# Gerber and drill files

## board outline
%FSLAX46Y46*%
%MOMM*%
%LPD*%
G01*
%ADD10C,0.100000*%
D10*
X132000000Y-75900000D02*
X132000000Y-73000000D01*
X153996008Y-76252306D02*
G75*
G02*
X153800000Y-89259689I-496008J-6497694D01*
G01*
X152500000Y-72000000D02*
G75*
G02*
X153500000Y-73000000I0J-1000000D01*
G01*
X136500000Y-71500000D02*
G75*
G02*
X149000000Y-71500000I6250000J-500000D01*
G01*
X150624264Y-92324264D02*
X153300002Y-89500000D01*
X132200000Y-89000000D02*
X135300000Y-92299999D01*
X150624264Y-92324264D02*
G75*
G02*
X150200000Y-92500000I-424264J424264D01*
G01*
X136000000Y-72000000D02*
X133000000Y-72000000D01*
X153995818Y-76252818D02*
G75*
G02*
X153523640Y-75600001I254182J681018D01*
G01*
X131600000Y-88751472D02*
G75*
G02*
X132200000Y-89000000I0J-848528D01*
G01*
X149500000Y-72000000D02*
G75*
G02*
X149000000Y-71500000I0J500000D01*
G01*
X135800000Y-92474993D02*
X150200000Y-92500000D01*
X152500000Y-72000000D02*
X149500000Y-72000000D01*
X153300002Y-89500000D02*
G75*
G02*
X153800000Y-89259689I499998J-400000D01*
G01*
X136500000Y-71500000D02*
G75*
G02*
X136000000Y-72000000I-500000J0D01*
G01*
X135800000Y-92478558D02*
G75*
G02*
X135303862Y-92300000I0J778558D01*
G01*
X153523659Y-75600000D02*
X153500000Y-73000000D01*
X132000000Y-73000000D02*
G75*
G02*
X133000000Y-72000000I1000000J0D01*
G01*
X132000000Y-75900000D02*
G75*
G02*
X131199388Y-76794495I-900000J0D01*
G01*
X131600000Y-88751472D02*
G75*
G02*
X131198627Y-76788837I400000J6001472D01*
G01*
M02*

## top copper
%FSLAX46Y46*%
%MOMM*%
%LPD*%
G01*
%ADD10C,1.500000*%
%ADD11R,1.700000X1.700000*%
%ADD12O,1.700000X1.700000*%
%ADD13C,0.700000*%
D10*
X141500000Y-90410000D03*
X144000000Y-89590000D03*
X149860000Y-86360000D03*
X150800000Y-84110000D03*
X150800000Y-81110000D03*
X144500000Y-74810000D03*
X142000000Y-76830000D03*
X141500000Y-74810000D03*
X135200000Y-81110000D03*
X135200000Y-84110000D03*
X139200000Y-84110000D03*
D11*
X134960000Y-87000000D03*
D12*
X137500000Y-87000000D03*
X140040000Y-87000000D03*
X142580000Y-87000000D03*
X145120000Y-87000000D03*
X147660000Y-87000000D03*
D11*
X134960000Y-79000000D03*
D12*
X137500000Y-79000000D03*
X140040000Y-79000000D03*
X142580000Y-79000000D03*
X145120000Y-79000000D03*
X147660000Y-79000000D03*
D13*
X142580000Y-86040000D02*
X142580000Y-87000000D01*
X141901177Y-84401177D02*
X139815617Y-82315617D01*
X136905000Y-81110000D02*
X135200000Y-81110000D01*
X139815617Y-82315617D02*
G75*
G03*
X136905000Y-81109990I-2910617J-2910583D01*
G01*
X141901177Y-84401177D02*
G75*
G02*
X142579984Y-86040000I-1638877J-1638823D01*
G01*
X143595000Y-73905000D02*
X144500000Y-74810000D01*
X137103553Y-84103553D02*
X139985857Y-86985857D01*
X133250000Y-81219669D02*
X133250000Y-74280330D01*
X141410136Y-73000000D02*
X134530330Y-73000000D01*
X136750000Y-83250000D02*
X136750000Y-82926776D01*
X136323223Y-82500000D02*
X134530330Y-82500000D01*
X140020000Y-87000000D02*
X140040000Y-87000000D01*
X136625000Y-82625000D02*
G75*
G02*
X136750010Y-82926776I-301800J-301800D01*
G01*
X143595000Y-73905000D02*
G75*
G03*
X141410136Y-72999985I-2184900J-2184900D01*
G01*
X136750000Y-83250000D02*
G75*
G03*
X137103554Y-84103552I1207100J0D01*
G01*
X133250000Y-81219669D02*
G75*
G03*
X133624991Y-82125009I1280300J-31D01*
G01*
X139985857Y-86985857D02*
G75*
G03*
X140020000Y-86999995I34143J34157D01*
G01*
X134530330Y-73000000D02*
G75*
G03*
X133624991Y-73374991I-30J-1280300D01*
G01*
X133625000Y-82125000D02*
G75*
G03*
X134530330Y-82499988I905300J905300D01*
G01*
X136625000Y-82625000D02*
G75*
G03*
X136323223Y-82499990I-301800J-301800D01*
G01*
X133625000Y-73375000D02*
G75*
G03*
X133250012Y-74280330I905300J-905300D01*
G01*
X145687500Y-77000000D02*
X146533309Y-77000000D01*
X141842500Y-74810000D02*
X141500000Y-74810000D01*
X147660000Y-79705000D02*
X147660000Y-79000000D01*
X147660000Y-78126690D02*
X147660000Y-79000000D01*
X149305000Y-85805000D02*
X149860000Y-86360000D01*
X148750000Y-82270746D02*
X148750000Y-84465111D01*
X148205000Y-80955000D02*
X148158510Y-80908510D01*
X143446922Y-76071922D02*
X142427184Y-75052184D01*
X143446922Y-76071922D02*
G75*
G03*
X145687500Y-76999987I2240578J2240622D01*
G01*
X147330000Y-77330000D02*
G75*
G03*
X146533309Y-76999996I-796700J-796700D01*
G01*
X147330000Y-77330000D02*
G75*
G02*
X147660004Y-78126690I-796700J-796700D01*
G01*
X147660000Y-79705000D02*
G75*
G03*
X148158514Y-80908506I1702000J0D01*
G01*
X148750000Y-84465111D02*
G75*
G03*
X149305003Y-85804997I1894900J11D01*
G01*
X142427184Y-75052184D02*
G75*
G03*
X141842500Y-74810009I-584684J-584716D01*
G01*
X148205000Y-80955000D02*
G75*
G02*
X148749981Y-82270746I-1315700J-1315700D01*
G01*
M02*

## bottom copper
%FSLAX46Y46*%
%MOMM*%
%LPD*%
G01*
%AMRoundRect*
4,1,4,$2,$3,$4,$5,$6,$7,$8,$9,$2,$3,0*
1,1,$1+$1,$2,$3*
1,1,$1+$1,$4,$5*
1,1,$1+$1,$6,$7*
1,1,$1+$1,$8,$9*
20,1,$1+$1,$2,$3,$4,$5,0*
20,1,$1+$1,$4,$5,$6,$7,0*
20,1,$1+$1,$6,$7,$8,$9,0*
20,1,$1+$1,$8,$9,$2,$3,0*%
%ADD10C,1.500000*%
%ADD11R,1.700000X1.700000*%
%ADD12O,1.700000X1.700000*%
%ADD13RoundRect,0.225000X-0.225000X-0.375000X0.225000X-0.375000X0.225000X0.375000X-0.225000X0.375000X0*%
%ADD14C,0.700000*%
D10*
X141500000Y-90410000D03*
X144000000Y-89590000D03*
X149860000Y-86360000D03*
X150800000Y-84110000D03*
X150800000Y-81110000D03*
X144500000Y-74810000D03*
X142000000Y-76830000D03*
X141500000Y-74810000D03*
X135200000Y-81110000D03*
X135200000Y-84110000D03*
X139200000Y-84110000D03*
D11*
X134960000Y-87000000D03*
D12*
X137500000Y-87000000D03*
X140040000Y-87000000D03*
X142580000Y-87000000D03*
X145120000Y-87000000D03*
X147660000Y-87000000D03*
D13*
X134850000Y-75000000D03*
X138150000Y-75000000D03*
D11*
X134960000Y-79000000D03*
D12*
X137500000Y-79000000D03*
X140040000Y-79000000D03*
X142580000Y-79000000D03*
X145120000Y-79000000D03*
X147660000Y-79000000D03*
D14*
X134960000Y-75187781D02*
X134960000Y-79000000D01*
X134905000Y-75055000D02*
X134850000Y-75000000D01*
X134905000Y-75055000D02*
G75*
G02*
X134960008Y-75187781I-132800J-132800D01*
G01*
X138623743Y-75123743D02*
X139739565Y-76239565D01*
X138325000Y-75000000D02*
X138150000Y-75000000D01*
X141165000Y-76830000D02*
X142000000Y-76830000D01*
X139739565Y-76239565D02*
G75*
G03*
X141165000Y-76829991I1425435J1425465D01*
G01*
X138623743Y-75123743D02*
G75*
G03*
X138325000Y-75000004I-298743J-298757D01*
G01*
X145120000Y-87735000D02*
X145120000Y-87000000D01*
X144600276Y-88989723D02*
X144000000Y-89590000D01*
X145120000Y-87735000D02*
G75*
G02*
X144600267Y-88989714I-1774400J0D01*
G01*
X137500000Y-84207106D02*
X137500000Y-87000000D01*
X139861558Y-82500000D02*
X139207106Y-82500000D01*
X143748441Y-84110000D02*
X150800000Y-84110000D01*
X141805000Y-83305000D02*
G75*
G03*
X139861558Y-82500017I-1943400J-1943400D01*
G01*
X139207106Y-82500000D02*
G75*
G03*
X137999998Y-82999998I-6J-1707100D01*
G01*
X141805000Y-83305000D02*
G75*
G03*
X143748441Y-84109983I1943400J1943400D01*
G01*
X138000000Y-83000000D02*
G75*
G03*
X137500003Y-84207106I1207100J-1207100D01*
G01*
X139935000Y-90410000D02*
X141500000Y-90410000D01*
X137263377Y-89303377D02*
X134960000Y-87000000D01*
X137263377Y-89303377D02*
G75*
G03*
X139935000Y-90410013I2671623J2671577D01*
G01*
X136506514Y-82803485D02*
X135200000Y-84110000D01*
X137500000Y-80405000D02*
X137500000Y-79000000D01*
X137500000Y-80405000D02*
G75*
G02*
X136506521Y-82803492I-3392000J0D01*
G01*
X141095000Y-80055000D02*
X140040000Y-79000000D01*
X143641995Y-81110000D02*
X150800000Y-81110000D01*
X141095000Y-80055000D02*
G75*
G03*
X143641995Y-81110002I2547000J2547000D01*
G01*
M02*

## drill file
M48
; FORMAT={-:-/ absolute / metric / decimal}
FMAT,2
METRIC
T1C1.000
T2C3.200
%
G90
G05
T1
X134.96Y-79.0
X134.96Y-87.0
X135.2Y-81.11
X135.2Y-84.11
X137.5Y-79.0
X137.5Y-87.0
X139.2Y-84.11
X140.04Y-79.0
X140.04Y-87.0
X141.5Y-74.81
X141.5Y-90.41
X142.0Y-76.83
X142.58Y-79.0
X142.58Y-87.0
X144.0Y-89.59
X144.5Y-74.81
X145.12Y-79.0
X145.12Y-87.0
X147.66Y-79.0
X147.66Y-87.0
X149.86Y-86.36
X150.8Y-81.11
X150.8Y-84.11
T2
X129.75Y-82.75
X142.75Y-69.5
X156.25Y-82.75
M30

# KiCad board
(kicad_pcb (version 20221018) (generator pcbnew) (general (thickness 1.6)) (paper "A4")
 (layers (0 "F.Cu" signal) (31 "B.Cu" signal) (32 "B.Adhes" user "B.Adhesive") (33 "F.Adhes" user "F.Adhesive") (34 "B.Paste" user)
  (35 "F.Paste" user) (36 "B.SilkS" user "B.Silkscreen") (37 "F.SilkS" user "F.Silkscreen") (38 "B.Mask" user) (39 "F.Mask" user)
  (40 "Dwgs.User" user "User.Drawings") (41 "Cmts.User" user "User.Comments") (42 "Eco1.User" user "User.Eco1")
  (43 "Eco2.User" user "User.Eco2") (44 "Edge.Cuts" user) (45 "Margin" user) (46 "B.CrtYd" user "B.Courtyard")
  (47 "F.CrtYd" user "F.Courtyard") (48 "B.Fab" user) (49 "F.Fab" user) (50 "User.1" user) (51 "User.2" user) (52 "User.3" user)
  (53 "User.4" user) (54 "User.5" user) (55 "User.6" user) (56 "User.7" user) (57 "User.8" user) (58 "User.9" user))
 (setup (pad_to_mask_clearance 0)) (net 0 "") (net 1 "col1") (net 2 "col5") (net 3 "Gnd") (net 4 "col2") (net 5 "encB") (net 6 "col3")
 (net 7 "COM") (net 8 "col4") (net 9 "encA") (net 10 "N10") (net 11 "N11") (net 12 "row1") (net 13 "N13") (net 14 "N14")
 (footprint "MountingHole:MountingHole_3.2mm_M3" (layer "F.Cu") (at 129.75 82.75)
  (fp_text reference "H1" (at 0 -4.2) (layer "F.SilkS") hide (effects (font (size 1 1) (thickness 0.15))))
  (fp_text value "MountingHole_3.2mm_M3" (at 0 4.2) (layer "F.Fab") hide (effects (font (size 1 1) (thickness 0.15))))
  (pad "" np_thru_hole circle (at 0 0) (size 3.2 3.2) (drill 3.2) (layers "*.Cu" "*.Mask")))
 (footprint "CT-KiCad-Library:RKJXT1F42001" (layer "F.Cu") (at 143 82.61)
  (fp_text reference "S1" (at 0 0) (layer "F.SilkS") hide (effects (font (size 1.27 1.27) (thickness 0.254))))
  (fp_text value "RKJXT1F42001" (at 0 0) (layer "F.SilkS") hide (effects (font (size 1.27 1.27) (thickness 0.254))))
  (pad "1" thru_hole circle (at -1.5 7.8) (size 1.5 1.5) (drill 1) (layers "*.Cu" "*.Mask") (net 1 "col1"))
  (pad "2" thru_hole circle (at 1 6.98) (size 1.5 1.5) (drill 1) (layers "*.Cu" "*.Mask") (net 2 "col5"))
  (pad "3" thru_hole circle (at 6.86 3.75) (size 1.5 1.5) (drill 1) (layers "*.Cu" "*.Mask") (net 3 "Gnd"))
  (pad "4" thru_hole circle (at 7.8 1.5) (size 1.5 1.5) (drill 1) (layers "*.Cu" "*.Mask") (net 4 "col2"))
  (pad "5" thru_hole circle (at 7.8 -1.5) (size 1.5 1.5) (drill 1) (layers "*.Cu" "*.Mask") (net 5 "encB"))
  (pad "6" thru_hole circle (at 1.5 -7.8) (size 1.5 1.5) (drill 1) (layers "*.Cu" "*.Mask") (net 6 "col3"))
  (pad "7" thru_hole circle (at -1 -5.78) (size 1.5 1.5) (drill 1) (layers "*.Cu" "*.Mask") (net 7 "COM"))
  (pad "8" thru_hole circle (at -1.5 -7.8) (size 1.5 1.5) (drill 1) (layers "*.Cu" "*.Mask") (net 3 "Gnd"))
  (pad "9" thru_hole circle (at -7.8 -1.5) (size 1.5 1.5) (drill 1) (layers "*.Cu" "*.Mask") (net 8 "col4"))
  (pad "10" thru_hole circle (at -7.8 1.5) (size 1.5 1.5) (drill 1) (layers "*.Cu" "*.Mask") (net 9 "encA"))
  (pad "11" thru_hole circle (at -3.8 1.5) (size 1.5 1.5) (drill 1) (layers "*.Cu" "*.Mask") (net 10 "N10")))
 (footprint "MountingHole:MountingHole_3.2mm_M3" (layer "F.Cu") (at 142.75 69.5)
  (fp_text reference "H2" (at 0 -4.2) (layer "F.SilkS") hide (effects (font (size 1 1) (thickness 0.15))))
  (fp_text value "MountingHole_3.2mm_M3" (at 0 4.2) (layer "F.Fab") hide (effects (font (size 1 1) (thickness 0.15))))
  (pad "" np_thru_hole circle (at 0 0) (size 3.2 3.2) (drill 3.2) (layers "*.Cu" "*.Mask")))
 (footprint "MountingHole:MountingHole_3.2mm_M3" (layer "F.Cu") (at 156.25 82.75)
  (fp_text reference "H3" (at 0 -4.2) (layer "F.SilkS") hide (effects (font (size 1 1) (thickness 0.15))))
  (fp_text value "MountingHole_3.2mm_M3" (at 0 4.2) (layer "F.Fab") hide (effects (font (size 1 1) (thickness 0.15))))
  (pad "" np_thru_hole circle (at 0 0) (size 3.2 3.2) (drill 3.2) (layers "*.Cu" "*.Mask")))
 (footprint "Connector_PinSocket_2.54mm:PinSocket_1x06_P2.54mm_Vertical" (layer "B.Cu") (at 134.96 87 -90)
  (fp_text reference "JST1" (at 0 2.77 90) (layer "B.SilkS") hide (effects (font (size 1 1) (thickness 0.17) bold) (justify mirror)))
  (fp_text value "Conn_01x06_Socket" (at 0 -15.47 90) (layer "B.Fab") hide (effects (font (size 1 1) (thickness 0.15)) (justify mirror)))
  (pad "1" thru_hole rect (at 0 0 270) (size 1.7 1.7) (drill 1) (layers "*.Cu" "*.Mask") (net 1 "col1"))
  (pad "2" thru_hole oval (at 0 -2.54 270) (size 1.7 1.7) (drill 1) (layers "*.Cu" "*.Mask") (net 4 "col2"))
  (pad "3" thru_hole oval (at 0 -5.08 270) (size 1.7 1.7) (drill 1) (layers "*.Cu" "*.Mask") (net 6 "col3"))
  (pad "4" thru_hole oval (at 0 -7.62 270) (size 1.7 1.7) (drill 1) (layers "*.Cu" "*.Mask") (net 8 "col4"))
  (pad "5" thru_hole oval (at 0 -10.16 270) (size 1.7 1.7) (drill 1) (layers "*.Cu" "*.Mask") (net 2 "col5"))
  (pad "6" thru_hole oval (at 0 -12.7 270) (size 1.7 1.7) (drill 1) (layers "*.Cu" "*.Mask") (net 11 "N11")))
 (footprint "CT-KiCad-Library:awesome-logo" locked (layer "B.Cu") (at 150.5 75 180)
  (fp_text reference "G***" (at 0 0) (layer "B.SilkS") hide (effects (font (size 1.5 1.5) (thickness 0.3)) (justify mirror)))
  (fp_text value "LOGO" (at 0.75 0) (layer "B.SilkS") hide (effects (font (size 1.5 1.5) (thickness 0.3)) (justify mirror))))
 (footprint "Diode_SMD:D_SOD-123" (layer "B.Cu") (at 136.5 75)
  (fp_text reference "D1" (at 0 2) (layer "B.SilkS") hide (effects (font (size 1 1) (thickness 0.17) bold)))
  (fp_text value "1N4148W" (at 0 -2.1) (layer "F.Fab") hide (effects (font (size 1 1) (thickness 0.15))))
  (pad "1" smd roundrect (at -1.65 0) (size 0.9 1.2) (layers "B.Cu" "B.Paste" "B.Mask") (roundrect_rratio 0.25) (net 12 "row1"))
  (pad "2" smd roundrect (at 1.65 0) (size 0.9 1.2) (layers "B.Cu" "B.Paste" "B.Mask") (roundrect_rratio 0.25) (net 7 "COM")))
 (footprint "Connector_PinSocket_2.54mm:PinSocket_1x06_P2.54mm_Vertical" (layer "B.Cu") (at 134.96 79 -90)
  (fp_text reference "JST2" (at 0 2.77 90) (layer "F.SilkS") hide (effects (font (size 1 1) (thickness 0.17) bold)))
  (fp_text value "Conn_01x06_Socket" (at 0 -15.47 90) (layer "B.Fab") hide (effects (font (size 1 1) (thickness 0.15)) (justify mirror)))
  (pad "1" thru_hole rect (at 0 0 270) (size 1.7 1.7) (drill 1) (layers "*.Cu" "*.Mask") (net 12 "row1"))
  (pad "2" thru_hole oval (at 0 -2.54 270) (size 1.7 1.7) (drill 1) (layers "*.Cu" "*.Mask") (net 9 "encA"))
  (pad "3" thru_hole oval (at 0 -5.08 270) (size 1.7 1.7) (drill 1) (layers "*.Cu" "*.Mask") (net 5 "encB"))
  (pad "4" thru_hole oval (at 0 -7.62 270) (size 1.7 1.7) (drill 1) (layers "*.Cu" "*.Mask") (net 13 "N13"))
  (pad "5" thru_hole oval (at 0 -10.16 270) (size 1.7 1.7) (drill 1) (layers "*.Cu" "*.Mask") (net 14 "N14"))
  (pad "6" thru_hole oval (at 0 -12.7 270) (size 1.7 1.7) (drill 1) (layers "*.Cu" "*.Mask") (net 3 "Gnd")))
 (gr_line (start 132 75.9) (end 132 73) (stroke (width 0.1) (type default)) (layer "Edge.Cuts"))
 (gr_arc (start 153.996008 76.252306) (mid 160.015858 82.848187) (end 153.8 89.259689) (stroke (width 0.1) (type default))
  (layer "Edge.Cuts"))
 (gr_arc (start 152.5 72) (mid 153.207107 72.292893) (end 153.5 73) (stroke (width 0.1) (type default)) (layer "Edge.Cuts"))
 (gr_arc (start 136.5 71.5) (mid 142.75 65.730032) (end 149 71.5) (stroke (width 0.1) (type default)) (layer "Edge.Cuts"))
 (gr_line (start 150.624264 92.324264) (end 153.300002 89.5) (stroke (width 0.1) (type default)) (layer "Edge.Cuts"))
 (gr_line (start 132.2 89) (end 135.3 92.299999) (stroke (width 0.1) (type default)) (layer "Edge.Cuts"))
 (gr_arc (start 150.624264 92.324264) (mid 150.42961 92.454328) (end 150.2 92.5) (stroke (width 0.1) (type default)) (layer "Edge.Cuts"))
 (gr_line (start 136 72) (end 133 72) (stroke (width 0.1) (type default)) (layer "Edge.Cuts"))
 (gr_arc (start 153.995818 76.252818) (mid 153.661019 75.997809) (end 153.523659 75.6) (stroke (width 0.1) (type default))
  (layer "Edge.Cuts"))
 (gr_arc (start 131.6 88.751472) (mid 131.924718 88.816062) (end 132.2 89) (stroke (width 0.1) (type default)) (layer "Edge.Cuts"))
 (gr_arc (start 149.5 72) (mid 149.146447 71.853553) (end 149 71.5) (stroke (width 0.1) (type default)) (layer "Edge.Cuts"))
 (gr_line (start 135.8 92.474993) (end 150.2 92.5) (stroke (width 0.1) (type default)) (layer "Edge.Cuts"))
 (gr_line (start 152.5 72) (end 149.5 72) (stroke (width 0.1) (type default)) (layer "Edge.Cuts"))
 (gr_arc (start 153.300002 89.5) (mid 153.522625 89.322885) (end 153.8 89.259689) (stroke (width 0.1) (type default)) (layer "Edge.Cuts"))
 (gr_arc (start 136.5 71.5) (mid 136.353553 71.853553) (end 136 72) (stroke (width 0.1) (type default)) (layer "Edge.Cuts"))
 (gr_arc (start 135.8 92.478558) (mid 135.536355 92.43256) (end 135.303862 92.3) (stroke (width 0.1) (type default)) (layer "Edge.Cuts"))
 (gr_line (start 153.523659 75.6) (end 153.5 73) (stroke (width 0.1) (type default)) (layer "Edge.Cuts"))
 (gr_arc (start 132 73) (mid 132.292893 72.292893) (end 133 72) (stroke (width 0.1) (type default)) (layer "Edge.Cuts"))
 (gr_arc (start 132 75.9) (mid 131.770615 76.500229) (end 131.199388 76.794495) (stroke (width 0.1) (type default)) (layer "Edge.Cuts"))
 (gr_arc (start 131.6 88.751472) (mid 125.988595 82.951696) (end 131.198627 76.788837) (stroke (width 0.1) (type default))
  (layer "Edge.Cuts"))
 (segment (start 134.96 75.187781) (end 134.96 79) (width 0.7) (layer "B.Cu") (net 12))
 (segment (start 134.905 75.055) (end 134.85 75) (width 0.7) (layer "B.Cu") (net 12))
 (arc (start 134.905 75.055) (mid 134.945705 75.11592) (end 134.96 75.187781) (width 0.7) (layer "B.Cu") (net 12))
 (segment (start 138.623743 75.123743) (end 139.739565 76.239565) (width 0.7) (layer "B.Cu") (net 7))
 (segment (start 138.325 75) (end 138.15 75) (width 0.7) (layer "B.Cu") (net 7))
 (segment (start 141.165 76.83) (end 142 76.83) (width 0.7) (layer "B.Cu") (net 7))
 (arc (start 139.739565 76.239565) (mid 140.39356 76.67655) (end 141.165 76.83) (width 0.7) (layer "B.Cu") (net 7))
 (arc (start 138.623743 75.123743) (mid 138.486678 75.032159) (end 138.325 75) (width 0.7) (layer "B.Cu") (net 7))
 (segment (start 145.12 87.735) (end 145.12 87) (width 0.7) (layer "B.Cu") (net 2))
 (segment (start 144.600276 88.989723) (end 144 89.59) (width 0.7) (layer "B.Cu") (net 2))
 (arc (start 145.12 87.735) (mid 144.984928 88.414051) (end 144.600276 88.989723) (width 0.7) (layer "B.Cu") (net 2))
 (segment (start 142.58 86.04) (end 142.58 87) (width 0.7) (layer "F.Cu") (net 8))
 (segment (start 141.901177 84.401177) (end 139.815617 82.315617) (width 0.7) (layer "F.Cu") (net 8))
 (segment (start 136.905 81.11) (end 135.2 81.11) (width 0.7) (layer "F.Cu") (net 8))
 (arc (start 139.815617 82.315617) (mid 138.480214 81.423329) (end 136.905 81.11) (width 0.7) (layer "F.Cu") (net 8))
 (arc (start 141.901177 84.401177) (mid 142.403579 85.153075) (end 142.58 86.04) (width 0.7) (layer "F.Cu") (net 8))
 (segment (start 143.595 73.905) (end 144.5 74.81) (width 0.7) (layer "F.Cu") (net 6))
 (segment (start 137.103553 84.103553) (end 139.985857 86.985857) (width 0.7) (layer "F.Cu") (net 6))
 (segment (start 133.25 81.219669) (end 133.25 74.28033) (width 0.7) (layer "F.Cu") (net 6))
 (segment (start 141.410136 73) (end 134.53033 73) (width 0.7) (layer "F.Cu") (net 6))
 (segment (start 136.75 83.25) (end 136.75 82.926776) (width 0.7) (layer "F.Cu") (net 6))
 (segment (start 136.323223 82.5) (end 134.53033 82.5) (width 0.7) (layer "F.Cu") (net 6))
 (segment (start 140.02 87) (end 140.04 87) (width 0.7) (layer "F.Cu") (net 6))
 (arc (start 136.625 82.625) (mid 136.717513 82.763456) (end 136.75 82.926776) (width 0.7) (layer "F.Cu") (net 6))
 (arc (start 143.595 73.905) (mid 142.592576 73.235201) (end 141.410136 73) (width 0.7) (layer "F.Cu") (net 6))
 (arc (start 136.75 83.25) (mid 136.841885 83.711939) (end 137.103553 84.103553) (width 0.7) (layer "F.Cu") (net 6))
 (arc (start 133.25 81.219669) (mid 133.347459 81.70963) (end 133.625 82.125) (width 0.7) (layer "F.Cu") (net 6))
 (arc (start 139.985857 86.985857) (mid 140.001522 86.996324) (end 140.02 87) (width 0.7) (layer "F.Cu") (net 6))
 (arc (start 134.53033 73) (mid 134.040368 73.097459) (end 133.625 73.375) (width 0.7) (layer "F.Cu") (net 6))
 (arc (start 133.625 82.125) (mid 134.040368 82.40254) (end 134.53033 82.5) (width 0.7) (layer "F.Cu") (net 6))
 (arc (start 136.625 82.625) (mid 136.486543 82.532486) (end 136.323223 82.5) (width 0.7) (layer "F.Cu") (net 6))
 (arc (start 133.625 73.375) (mid 133.347459 73.790368) (end 133.25 74.28033) (width 0.7) (layer "F.Cu") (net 6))
 (segment (start 137.5 84.207106) (end 137.5 87) (width 0.7) (layer "B.Cu") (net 4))
 (segment (start 139.861558 82.5) (end 139.207106 82.5) (width 0.7) (layer "B.Cu") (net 4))
 (segment (start 143.748441 84.11) (end 150.8 84.11) (width 0.7) (layer "B.Cu") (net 4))
 (arc (start 141.805 83.305) (mid 140.913341 82.709212) (end 139.861558 82.5) (width 0.7) (layer "B.Cu") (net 4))
 (arc (start 139.207106 82.5) (mid 138.553825 82.629945) (end 138 83) (width 0.7) (layer "B.Cu") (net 4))
 (arc (start 141.805 83.305) (mid 142.696658 83.900787) (end 143.748441 84.11) (width 0.7) (layer "B.Cu") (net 4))
 (arc (start 138 83) (mid 137.629945 83.553825) (end 137.5 84.207106) (width 0.7) (layer "B.Cu") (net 4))
 (segment (start 139.935 90.41) (end 141.5 90.41) (width 0.7) (layer "B.Cu") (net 1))
 (segment (start 137.263377 89.303377) (end 134.96 87) (width 0.7) (layer "B.Cu") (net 1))
 (arc (start 137.263377 89.303377) (mid 138.489128 90.122398) (end 139.935 90.41) (width 0.7) (layer "B.Cu") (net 1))
 (segment (start 136.506514 82.803485) (end 135.2 84.11) (width 0.7) (layer "B.Cu") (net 9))
 (segment (start 137.5 80.405) (end 137.5 79) (width 0.7) (layer "B.Cu") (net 9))
 (arc (start 137.5 80.405) (mid 137.241801 81.70305) (end 136.506514 82.803485) (width 0.7) (layer "B.Cu") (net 9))
 (segment (start 141.095 80.055) (end 140.04 79) (width 0.7) (layer "B.Cu") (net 5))
 (segment (start 143.641995 81.11) (end 150.8 81.11) (width 0.7) (layer "B.Cu") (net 5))
 (arc (start 141.095 80.055) (mid 142.263571 80.835814) (end 143.641995 81.11) (width 0.7) (layer "B.Cu") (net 5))
 (segment (start 145.6875 77) (end 146.533309 77) (width 0.7) (layer "F.Cu") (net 3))
 (segment (start 141.8425 74.81) (end 141.5 74.81) (width 0.7) (layer "F.Cu") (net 3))
 (segment (start 147.66 79.705) (end 147.66 79) (width 0.7) (layer "F.Cu") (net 3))
 (segment (start 147.66 78.12669) (end 147.66 79) (width 0.7) (layer "F.Cu") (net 3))
 (segment (start 149.305 85.805) (end 149.86 86.36) (width 0.7) (layer "F.Cu") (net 3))
 (segment (start 148.75 82.270746) (end 148.75 84.465111) (width 0.7) (layer "F.Cu") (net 3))
 (segment (start 148.205 80.955) (end 148.15851 80.90851) (width 0.7) (layer "F.Cu") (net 3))
 (segment (start 143.446922 76.071922) (end 142.427184 75.052184) (width 0.7) (layer "F.Cu") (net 3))
 (arc (start 143.446922 76.071922) (mid 144.474908 76.7588) (end 145.6875 77) (width 0.7) (layer "F.Cu") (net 3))
 (arc (start 147.33 77.33) (mid 146.964475 77.085764) (end 146.533309 77) (width 0.7) (layer "F.Cu") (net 3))
 (arc (start 147.33 77.33) (mid 147.574235 77.695524) (end 147.66 78.12669) (width 0.7) (layer "F.Cu") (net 3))
 (arc (start 147.66 79.705) (mid 147.789558 80.356334) (end 148.15851 80.90851) (width 0.7) (layer "F.Cu") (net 3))
 (arc (start 148.75 84.465111) (mid 148.894239 85.190253) (end 149.305 85.805) (width 0.7) (layer "F.Cu") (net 3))
 (arc (start 142.427184 75.052184) (mid 142.158928 74.872941) (end 141.8425 74.81) (width 0.7) (layer "F.Cu") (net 3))
 (arc (start 148.205 80.955) (mid 148.608359 81.558669) (end 148.75 82.270746) (width 0.7) (layer "F.Cu") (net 3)))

